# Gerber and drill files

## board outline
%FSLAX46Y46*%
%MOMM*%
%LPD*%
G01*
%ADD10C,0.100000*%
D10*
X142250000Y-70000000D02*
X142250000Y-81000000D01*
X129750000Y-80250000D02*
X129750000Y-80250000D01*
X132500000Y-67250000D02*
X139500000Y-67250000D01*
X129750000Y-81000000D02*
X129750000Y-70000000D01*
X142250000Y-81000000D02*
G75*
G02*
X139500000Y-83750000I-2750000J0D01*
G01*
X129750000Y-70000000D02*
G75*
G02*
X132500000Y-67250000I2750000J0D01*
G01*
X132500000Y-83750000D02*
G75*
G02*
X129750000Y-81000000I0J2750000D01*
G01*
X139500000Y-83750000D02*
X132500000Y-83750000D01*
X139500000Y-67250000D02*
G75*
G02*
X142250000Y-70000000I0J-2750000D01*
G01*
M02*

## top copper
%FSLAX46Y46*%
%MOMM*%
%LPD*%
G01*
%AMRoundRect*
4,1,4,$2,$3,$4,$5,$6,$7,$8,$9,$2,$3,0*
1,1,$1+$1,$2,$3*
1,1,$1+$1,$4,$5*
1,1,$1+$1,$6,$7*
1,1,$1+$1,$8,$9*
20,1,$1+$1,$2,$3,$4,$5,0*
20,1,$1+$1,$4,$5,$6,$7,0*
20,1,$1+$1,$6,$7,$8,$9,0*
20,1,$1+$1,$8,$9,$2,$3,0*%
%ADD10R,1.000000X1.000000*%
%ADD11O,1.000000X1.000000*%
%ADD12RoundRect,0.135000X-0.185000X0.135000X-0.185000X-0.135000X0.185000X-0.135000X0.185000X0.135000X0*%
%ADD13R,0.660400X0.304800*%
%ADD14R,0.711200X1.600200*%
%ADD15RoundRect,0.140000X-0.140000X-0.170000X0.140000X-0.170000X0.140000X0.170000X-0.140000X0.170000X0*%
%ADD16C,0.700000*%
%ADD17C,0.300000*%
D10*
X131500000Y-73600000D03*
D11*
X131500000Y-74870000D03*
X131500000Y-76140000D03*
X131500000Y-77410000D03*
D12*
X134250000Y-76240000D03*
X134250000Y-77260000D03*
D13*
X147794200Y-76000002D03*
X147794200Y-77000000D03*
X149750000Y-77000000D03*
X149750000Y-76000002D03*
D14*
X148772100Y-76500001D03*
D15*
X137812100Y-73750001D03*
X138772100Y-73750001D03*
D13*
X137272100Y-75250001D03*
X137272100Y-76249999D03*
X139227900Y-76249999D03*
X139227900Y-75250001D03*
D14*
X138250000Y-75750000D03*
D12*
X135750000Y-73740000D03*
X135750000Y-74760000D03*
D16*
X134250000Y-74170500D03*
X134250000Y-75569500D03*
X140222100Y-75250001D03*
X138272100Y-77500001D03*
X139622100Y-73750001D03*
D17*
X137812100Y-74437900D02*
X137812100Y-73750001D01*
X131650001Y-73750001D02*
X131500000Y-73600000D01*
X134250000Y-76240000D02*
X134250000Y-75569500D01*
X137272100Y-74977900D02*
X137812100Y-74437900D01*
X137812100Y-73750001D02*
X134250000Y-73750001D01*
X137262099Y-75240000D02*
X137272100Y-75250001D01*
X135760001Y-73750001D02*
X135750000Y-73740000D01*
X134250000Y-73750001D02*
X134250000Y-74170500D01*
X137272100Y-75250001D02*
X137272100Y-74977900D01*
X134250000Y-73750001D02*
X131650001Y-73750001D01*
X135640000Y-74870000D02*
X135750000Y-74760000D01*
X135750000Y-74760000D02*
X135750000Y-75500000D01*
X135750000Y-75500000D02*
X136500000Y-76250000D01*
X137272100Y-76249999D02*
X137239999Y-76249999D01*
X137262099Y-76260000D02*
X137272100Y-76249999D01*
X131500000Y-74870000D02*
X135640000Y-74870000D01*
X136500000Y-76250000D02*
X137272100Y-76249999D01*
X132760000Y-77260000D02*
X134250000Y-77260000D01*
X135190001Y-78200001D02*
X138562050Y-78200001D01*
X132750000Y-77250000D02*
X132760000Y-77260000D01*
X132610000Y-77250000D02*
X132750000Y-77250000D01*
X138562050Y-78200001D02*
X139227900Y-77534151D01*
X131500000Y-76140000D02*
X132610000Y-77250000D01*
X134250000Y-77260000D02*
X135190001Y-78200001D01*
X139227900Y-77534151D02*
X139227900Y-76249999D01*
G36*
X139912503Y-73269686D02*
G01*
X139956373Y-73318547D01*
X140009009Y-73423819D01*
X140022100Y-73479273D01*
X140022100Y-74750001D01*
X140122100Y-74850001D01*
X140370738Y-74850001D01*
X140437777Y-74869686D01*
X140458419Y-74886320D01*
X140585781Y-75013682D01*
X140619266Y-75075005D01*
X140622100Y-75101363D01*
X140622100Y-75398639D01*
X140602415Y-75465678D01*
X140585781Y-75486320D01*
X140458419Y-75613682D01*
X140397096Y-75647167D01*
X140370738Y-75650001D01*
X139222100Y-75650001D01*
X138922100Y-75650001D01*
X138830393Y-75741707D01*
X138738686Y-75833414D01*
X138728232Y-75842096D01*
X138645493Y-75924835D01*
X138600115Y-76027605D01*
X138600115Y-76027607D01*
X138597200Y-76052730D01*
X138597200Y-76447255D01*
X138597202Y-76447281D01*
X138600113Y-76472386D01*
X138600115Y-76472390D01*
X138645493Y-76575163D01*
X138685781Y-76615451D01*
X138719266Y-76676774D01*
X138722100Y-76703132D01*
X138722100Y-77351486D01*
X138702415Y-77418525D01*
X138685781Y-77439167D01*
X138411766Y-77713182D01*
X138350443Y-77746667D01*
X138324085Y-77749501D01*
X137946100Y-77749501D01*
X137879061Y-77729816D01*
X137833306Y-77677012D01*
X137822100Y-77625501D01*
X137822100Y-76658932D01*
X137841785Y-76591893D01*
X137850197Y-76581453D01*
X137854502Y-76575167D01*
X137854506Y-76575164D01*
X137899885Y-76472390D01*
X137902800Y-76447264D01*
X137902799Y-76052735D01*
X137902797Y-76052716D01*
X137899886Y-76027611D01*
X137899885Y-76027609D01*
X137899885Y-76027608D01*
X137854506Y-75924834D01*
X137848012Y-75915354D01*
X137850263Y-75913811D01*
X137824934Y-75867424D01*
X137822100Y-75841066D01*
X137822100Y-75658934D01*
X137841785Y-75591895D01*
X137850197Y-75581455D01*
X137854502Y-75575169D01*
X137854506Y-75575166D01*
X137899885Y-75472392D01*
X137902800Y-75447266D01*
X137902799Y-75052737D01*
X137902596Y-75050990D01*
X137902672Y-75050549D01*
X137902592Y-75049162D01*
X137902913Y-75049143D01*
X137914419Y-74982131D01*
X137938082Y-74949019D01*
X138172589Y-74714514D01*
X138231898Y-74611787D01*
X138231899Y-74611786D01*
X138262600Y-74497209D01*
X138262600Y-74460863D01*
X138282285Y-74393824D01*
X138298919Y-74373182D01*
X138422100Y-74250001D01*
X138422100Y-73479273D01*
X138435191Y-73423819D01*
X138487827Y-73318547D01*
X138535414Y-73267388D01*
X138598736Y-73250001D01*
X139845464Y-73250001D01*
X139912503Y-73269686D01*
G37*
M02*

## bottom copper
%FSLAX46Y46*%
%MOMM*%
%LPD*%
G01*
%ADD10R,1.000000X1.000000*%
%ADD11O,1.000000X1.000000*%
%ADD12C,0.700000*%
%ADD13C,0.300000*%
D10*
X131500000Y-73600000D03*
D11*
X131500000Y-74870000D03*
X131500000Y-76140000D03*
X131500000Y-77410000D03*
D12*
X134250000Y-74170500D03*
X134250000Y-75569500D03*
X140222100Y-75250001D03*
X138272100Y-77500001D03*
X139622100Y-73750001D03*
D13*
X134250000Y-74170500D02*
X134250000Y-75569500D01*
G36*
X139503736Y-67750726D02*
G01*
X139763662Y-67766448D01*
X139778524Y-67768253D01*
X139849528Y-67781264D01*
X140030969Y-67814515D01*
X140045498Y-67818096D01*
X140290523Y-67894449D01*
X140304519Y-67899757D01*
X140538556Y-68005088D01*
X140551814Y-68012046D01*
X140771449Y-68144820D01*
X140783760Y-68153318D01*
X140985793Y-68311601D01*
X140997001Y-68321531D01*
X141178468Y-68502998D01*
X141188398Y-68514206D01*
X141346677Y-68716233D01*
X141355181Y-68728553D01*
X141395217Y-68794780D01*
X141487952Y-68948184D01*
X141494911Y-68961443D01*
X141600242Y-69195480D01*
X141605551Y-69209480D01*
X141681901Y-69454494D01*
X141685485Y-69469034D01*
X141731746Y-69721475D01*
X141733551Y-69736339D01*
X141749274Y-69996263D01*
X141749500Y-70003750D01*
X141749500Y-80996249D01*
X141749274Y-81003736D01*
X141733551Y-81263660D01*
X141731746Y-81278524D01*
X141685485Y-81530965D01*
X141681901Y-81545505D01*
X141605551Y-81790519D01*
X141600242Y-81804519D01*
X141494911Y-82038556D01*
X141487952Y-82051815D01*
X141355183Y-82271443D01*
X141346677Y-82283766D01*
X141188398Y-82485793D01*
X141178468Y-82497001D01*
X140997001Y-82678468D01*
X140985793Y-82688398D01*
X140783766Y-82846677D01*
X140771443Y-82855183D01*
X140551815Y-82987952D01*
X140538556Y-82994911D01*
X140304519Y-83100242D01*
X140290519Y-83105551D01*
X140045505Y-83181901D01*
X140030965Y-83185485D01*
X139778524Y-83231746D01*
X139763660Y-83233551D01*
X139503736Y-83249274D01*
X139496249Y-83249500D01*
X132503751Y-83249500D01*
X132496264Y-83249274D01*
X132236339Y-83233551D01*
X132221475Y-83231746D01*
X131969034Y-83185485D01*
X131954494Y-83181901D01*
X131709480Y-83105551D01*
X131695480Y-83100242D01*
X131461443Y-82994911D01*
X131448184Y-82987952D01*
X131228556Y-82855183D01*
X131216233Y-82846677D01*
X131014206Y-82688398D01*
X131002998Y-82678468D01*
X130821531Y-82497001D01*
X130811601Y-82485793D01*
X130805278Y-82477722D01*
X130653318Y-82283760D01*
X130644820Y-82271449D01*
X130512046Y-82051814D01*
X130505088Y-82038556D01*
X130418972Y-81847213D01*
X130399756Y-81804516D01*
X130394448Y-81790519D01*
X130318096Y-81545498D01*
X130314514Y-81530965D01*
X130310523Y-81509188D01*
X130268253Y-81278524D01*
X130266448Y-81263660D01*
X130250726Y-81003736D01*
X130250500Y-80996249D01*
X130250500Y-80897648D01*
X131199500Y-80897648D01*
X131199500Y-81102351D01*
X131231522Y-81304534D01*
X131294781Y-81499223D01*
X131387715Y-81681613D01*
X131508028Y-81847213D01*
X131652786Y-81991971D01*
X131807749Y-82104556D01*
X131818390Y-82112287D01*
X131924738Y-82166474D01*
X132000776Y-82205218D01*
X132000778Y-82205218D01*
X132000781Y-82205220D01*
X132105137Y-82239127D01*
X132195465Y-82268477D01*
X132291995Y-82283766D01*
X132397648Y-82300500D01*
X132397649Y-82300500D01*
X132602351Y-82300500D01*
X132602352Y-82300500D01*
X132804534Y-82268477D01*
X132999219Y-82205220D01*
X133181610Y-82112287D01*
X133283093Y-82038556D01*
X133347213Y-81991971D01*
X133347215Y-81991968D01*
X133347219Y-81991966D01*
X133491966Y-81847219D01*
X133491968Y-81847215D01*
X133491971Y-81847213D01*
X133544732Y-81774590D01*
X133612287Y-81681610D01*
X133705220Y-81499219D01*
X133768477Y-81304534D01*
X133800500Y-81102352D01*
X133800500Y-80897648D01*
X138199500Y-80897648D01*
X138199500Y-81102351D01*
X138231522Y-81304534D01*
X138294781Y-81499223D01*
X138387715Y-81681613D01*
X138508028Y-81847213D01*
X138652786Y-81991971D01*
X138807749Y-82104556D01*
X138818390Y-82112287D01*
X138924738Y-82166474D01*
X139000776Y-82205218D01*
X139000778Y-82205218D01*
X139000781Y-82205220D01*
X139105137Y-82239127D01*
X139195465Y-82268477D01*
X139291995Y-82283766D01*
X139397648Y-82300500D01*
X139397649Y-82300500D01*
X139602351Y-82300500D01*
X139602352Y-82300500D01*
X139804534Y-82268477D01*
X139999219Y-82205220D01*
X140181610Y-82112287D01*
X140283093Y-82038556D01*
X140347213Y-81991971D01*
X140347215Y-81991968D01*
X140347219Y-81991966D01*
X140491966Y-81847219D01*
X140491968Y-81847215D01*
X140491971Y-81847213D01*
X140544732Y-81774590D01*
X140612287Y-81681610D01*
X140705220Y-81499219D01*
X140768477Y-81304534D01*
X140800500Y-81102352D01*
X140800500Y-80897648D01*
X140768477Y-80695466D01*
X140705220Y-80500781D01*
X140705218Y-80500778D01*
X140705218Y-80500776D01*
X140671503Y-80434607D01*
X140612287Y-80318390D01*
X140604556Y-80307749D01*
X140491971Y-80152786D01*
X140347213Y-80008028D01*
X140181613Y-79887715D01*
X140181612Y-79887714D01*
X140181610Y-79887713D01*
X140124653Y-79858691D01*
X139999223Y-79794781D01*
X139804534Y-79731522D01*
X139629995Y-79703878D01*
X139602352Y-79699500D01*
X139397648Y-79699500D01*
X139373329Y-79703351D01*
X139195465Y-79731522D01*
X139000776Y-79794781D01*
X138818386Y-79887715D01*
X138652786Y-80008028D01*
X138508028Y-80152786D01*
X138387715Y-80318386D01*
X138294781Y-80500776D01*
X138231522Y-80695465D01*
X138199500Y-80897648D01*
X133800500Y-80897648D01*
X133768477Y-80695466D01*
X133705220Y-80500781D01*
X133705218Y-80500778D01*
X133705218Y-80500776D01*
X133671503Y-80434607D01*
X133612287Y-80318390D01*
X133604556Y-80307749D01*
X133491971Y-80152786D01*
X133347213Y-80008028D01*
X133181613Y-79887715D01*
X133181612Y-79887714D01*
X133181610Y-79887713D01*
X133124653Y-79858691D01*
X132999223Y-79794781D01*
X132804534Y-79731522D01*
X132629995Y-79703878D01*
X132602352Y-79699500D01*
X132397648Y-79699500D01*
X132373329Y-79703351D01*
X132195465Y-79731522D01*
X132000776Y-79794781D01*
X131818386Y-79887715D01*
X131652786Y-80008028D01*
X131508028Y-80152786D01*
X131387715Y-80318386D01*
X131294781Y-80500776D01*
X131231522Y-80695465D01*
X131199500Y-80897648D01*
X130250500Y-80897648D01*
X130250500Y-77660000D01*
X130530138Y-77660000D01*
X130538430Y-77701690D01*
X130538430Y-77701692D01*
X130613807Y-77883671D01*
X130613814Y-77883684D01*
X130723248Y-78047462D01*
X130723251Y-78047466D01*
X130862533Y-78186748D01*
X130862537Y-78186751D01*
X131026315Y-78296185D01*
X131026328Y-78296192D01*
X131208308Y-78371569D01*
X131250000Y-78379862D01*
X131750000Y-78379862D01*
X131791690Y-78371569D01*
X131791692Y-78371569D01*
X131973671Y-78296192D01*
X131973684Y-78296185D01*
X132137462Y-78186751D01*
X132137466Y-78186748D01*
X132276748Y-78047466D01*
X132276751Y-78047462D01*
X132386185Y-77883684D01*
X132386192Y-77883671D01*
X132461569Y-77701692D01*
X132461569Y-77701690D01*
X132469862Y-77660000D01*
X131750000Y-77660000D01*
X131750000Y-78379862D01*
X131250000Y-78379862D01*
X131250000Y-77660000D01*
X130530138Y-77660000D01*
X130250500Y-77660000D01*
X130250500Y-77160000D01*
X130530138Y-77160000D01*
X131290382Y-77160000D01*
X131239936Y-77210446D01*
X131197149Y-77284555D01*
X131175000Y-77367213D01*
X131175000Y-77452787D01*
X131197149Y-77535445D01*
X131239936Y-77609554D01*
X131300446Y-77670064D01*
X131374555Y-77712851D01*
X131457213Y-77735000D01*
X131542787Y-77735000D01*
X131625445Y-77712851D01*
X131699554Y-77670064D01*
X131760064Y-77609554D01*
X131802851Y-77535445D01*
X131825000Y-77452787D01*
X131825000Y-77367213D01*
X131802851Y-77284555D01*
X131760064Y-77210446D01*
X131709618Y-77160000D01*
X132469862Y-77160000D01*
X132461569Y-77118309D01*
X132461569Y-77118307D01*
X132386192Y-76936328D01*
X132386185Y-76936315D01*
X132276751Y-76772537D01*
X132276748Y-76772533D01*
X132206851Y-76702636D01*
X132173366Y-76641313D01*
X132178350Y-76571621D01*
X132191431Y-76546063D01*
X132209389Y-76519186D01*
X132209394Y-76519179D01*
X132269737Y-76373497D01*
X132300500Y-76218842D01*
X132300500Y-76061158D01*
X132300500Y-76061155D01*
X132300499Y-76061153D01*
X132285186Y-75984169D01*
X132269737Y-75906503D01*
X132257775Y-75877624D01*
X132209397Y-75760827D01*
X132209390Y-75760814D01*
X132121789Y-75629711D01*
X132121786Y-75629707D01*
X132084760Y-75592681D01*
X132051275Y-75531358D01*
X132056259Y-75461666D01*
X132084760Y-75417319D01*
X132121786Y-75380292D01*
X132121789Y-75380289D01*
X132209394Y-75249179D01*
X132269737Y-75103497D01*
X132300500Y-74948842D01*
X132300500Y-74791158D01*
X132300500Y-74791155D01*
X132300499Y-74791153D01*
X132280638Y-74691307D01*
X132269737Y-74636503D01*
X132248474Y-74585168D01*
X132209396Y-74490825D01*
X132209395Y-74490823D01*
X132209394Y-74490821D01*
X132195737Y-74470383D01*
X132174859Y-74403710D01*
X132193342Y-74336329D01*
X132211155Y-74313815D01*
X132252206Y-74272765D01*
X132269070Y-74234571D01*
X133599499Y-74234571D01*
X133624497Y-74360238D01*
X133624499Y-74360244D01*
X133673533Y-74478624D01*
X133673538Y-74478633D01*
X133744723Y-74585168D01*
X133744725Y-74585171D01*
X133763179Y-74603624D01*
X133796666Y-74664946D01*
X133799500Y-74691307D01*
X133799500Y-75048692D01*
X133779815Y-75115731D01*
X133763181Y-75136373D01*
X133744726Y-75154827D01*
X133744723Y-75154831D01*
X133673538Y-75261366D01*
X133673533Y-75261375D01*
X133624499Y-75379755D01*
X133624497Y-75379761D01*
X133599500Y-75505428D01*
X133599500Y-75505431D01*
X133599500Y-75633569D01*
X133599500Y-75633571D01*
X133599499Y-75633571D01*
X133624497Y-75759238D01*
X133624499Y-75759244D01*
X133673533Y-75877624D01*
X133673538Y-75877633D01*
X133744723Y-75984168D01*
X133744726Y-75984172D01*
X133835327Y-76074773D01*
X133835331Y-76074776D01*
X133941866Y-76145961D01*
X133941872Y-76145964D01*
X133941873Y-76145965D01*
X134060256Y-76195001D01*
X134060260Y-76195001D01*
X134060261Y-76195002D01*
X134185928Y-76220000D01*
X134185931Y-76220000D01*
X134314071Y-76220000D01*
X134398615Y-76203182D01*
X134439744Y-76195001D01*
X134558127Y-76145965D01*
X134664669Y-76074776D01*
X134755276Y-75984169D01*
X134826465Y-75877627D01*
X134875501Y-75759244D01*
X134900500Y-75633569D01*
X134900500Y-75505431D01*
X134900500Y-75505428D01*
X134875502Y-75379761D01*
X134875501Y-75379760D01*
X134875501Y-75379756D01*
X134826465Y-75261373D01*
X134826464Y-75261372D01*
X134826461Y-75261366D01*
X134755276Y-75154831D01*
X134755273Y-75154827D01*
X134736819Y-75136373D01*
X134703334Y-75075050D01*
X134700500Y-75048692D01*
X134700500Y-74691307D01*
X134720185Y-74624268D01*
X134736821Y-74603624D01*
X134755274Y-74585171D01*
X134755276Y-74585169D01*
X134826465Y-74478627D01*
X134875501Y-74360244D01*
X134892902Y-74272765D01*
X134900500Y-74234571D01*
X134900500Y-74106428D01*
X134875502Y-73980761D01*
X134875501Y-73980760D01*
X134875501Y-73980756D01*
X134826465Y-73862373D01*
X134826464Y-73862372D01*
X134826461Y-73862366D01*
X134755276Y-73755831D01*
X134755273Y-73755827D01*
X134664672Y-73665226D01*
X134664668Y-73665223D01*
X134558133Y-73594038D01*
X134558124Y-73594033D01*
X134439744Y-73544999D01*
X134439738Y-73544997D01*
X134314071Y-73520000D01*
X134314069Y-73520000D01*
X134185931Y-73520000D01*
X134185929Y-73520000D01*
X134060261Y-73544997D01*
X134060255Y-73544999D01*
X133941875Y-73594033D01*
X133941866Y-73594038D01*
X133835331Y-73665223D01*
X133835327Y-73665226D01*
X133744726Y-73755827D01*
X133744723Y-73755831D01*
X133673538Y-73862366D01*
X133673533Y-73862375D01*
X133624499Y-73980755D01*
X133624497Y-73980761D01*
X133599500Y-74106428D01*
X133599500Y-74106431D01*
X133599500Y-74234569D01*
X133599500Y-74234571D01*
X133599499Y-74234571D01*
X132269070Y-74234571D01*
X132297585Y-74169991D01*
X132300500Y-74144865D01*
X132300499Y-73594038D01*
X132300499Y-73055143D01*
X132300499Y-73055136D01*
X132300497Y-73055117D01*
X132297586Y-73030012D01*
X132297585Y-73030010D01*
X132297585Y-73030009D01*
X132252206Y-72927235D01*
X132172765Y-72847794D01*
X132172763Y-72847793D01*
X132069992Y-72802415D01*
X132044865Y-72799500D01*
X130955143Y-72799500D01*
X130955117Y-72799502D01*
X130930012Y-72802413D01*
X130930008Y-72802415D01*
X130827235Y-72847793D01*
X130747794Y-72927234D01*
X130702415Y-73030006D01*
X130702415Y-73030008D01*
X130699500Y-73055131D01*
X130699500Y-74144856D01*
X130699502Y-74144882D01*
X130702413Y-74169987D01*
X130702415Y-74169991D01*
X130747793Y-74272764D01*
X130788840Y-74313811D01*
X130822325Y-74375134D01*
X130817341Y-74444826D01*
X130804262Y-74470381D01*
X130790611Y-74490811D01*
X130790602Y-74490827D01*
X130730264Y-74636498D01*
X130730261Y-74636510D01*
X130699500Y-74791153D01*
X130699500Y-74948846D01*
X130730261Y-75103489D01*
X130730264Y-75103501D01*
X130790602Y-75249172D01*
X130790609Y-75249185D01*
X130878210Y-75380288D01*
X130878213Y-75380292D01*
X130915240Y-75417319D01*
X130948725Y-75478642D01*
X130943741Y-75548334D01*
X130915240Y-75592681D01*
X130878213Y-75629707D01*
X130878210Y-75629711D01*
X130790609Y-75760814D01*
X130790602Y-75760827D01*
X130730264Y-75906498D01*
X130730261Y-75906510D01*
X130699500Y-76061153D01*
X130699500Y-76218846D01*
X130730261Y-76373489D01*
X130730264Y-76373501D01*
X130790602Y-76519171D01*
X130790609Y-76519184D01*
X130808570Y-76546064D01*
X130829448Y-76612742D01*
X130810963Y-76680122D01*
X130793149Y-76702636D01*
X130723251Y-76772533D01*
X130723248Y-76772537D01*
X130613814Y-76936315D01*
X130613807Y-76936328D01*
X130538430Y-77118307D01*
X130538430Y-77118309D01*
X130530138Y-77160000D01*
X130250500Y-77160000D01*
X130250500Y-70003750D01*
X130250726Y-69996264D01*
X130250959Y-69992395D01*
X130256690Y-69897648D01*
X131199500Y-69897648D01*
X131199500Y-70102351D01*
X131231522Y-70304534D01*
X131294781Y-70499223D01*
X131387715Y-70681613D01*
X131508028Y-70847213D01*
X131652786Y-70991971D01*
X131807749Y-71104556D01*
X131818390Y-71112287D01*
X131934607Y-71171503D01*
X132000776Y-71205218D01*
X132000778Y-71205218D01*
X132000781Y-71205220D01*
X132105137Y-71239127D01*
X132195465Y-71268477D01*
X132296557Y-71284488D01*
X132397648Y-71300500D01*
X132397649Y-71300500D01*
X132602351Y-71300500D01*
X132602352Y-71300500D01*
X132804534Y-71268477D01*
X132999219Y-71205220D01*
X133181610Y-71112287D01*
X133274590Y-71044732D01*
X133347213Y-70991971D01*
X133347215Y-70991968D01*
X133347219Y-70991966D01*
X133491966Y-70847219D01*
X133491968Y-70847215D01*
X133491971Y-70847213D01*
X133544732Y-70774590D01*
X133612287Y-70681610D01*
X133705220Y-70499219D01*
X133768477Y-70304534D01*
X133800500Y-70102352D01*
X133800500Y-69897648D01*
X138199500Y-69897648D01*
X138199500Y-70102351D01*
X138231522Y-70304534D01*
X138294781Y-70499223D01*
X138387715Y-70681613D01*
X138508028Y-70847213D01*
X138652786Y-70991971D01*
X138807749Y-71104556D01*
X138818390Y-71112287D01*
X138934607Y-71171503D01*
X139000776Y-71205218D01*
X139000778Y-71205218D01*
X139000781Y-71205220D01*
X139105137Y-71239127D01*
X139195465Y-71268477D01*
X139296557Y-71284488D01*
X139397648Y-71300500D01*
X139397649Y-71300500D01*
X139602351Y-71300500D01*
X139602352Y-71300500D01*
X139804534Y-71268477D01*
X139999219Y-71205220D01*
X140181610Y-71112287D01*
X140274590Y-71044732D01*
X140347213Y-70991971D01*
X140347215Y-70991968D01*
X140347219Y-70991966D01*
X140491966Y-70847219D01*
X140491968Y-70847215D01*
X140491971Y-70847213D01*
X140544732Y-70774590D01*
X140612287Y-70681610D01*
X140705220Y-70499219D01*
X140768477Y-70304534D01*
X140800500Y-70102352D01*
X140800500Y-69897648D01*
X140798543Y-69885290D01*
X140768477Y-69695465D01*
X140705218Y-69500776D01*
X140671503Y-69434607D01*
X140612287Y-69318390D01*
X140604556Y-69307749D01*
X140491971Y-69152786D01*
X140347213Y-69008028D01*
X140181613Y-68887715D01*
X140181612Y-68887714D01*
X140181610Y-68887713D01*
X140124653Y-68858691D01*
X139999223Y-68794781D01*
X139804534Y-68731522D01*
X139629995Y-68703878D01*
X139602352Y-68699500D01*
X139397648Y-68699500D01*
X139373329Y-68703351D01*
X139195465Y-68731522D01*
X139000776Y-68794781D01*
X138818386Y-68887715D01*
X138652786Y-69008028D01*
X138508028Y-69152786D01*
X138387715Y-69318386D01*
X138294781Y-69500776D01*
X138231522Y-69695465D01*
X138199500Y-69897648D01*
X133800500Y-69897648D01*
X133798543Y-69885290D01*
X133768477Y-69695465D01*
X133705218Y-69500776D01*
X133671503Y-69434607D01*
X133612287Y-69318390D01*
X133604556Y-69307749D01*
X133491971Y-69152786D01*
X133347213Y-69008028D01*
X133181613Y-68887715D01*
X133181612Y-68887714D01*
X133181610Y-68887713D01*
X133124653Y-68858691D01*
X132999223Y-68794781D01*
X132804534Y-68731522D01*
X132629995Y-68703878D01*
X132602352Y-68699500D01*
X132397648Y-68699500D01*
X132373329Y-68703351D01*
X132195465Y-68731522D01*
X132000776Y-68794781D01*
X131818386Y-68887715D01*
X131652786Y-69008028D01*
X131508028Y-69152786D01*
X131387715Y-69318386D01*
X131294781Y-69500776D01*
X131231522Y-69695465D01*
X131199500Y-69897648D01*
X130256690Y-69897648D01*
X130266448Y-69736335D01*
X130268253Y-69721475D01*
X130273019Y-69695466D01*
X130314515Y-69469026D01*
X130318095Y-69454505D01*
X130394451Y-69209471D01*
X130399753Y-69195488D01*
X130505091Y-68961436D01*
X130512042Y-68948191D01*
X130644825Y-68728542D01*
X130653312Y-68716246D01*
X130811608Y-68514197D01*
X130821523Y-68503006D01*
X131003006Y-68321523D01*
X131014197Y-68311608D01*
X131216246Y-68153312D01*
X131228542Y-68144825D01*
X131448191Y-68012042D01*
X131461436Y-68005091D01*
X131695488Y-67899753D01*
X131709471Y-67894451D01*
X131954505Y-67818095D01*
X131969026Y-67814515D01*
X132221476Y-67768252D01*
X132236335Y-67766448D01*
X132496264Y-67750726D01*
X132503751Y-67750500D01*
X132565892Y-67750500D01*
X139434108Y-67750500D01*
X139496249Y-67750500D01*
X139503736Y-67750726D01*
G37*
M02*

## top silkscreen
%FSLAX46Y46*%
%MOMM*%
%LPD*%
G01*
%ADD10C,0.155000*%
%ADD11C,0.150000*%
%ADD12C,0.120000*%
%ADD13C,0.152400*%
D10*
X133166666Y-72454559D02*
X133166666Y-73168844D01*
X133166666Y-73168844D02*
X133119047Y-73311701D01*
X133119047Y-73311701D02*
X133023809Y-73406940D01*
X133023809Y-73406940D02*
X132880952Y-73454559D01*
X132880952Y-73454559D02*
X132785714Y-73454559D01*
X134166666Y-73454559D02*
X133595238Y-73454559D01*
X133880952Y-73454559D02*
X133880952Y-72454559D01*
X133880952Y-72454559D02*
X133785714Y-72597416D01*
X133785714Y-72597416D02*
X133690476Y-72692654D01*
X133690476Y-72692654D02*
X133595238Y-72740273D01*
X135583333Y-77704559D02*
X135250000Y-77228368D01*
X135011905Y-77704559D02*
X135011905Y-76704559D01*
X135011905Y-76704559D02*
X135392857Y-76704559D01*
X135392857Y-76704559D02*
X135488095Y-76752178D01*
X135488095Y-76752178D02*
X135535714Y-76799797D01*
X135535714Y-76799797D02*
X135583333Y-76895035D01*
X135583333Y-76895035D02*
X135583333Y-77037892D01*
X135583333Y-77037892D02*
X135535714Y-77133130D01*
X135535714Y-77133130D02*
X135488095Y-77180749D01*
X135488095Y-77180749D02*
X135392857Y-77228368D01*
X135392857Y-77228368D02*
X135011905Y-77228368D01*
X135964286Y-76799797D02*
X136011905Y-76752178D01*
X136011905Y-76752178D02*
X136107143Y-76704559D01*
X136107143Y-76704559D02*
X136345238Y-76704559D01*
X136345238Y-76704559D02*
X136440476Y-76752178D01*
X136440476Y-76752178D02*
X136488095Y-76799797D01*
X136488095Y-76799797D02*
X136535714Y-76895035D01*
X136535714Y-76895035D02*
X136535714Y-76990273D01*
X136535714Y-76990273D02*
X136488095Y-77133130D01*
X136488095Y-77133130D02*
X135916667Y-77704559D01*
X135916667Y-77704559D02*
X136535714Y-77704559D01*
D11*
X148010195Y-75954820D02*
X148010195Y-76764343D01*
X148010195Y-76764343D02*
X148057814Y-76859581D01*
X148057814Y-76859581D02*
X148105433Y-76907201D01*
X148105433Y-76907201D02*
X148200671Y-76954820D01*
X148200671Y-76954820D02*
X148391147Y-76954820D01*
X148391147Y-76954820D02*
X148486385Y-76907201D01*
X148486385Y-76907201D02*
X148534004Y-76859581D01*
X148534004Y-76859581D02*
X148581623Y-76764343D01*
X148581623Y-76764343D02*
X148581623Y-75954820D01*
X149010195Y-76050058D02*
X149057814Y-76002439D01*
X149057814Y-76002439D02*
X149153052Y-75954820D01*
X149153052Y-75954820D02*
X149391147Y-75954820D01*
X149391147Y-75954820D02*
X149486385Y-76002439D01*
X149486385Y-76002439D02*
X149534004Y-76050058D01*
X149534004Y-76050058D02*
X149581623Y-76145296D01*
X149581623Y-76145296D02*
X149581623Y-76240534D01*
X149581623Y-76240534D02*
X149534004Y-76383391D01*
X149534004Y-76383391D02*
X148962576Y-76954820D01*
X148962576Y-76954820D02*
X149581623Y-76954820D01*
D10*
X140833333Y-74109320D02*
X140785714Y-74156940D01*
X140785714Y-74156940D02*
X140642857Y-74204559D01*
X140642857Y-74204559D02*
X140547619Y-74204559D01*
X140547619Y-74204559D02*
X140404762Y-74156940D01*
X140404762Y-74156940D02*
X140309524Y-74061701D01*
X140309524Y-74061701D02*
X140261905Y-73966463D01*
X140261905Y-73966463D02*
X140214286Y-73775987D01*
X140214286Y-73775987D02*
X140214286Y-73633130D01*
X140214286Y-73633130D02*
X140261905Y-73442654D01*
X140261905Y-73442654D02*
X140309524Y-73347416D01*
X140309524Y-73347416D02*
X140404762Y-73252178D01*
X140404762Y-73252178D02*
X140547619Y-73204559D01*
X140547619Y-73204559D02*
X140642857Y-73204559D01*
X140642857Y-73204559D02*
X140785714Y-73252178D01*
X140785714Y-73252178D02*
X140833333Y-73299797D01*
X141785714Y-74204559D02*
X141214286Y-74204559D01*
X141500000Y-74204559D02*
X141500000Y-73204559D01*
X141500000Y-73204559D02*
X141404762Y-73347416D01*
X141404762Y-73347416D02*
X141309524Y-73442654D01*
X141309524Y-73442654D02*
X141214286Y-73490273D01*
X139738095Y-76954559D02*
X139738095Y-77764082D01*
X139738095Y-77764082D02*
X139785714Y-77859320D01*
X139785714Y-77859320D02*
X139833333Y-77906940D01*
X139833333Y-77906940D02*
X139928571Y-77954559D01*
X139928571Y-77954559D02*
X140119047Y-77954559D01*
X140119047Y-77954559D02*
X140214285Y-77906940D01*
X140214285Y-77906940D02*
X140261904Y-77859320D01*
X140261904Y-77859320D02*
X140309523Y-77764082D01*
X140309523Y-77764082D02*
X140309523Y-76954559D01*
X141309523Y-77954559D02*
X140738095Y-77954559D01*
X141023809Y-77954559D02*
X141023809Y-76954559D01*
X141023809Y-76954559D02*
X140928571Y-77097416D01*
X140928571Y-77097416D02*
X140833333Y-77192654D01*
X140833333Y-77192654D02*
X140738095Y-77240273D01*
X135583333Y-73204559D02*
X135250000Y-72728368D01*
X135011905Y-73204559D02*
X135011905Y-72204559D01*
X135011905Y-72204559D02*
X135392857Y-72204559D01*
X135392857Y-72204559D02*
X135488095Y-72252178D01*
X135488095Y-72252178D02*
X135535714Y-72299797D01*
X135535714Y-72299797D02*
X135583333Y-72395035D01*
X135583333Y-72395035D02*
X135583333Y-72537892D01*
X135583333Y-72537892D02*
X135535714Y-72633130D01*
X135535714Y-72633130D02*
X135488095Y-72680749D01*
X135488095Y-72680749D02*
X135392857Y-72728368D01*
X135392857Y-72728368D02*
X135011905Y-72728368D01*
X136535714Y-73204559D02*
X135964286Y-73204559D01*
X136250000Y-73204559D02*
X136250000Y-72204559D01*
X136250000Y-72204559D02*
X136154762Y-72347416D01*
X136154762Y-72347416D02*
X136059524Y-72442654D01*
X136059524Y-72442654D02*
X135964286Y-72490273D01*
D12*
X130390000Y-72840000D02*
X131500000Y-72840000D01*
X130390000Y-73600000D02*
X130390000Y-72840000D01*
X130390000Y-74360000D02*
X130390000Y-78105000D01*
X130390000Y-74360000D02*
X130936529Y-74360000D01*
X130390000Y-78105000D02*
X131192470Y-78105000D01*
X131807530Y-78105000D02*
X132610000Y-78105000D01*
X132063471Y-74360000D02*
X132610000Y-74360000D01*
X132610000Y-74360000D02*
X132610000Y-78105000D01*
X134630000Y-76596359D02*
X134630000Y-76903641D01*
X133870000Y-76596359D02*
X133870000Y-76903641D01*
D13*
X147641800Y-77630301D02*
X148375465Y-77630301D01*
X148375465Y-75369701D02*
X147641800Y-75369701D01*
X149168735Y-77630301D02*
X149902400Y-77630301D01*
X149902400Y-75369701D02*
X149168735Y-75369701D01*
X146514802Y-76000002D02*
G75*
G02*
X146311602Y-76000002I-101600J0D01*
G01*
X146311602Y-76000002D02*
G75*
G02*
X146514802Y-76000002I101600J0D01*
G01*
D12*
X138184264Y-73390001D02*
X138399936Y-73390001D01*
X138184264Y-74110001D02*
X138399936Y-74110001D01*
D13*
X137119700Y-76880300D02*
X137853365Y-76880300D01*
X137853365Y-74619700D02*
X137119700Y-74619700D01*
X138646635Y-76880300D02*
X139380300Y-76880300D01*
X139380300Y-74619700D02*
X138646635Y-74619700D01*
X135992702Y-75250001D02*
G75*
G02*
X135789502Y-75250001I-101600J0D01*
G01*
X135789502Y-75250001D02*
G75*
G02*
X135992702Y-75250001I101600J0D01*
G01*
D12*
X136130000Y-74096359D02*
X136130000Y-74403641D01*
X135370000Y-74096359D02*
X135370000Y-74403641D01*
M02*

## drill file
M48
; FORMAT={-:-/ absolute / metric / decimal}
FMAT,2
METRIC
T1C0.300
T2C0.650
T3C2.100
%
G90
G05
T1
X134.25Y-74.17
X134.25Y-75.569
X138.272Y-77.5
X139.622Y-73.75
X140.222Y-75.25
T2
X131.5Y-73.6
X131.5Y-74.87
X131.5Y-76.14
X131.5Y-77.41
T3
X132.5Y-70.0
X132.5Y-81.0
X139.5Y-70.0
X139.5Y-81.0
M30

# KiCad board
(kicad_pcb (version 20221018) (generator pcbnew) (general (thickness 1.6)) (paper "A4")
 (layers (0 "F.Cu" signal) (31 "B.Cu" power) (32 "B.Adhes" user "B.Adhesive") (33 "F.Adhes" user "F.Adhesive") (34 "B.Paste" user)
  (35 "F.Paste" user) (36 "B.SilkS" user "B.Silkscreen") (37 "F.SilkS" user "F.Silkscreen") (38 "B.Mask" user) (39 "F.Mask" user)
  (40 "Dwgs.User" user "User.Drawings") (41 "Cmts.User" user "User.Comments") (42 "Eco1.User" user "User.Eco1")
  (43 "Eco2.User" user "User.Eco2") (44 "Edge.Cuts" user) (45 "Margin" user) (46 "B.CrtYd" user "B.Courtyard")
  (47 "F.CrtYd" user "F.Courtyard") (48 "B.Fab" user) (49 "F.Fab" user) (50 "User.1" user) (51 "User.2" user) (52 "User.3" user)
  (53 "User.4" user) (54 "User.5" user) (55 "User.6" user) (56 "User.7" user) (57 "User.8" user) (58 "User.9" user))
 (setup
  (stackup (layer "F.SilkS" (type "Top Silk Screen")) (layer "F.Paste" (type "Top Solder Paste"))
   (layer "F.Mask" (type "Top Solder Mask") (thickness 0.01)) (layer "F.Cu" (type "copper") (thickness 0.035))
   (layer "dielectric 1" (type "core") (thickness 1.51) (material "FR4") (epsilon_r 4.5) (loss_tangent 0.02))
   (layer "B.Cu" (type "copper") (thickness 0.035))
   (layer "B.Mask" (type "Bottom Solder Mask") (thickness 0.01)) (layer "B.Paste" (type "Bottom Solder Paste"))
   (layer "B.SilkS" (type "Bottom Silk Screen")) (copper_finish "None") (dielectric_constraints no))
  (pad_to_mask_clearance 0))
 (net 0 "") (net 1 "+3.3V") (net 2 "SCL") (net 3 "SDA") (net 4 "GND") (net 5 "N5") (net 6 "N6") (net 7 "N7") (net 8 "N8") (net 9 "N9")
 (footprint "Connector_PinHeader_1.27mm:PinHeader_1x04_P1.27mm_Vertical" (layer "F.Cu") (at 131.5 73.6)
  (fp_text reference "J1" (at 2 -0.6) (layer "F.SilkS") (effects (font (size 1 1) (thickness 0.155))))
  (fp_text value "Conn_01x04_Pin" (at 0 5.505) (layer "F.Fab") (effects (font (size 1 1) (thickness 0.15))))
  (fp_line (start -1.11 -0.76) (end 0 -0.76) (stroke (width 0.12) (type solid)) (layer "F.SilkS"))
  (fp_line (start -1.11 0) (end -1.11 -0.76) (stroke (width 0.12) (type solid)) (layer "F.SilkS"))
  (fp_line (start -1.11 0.76) (end -1.11 4.505) (stroke (width 0.12) (type solid)) (layer "F.SilkS"))
  (fp_line (start -1.11 0.76) (end -0.563471 0.76) (stroke (width 0.12) (type solid)) (layer "F.SilkS"))
  (fp_line (start -1.11 4.505) (end -0.30753 4.505) (stroke (width 0.12) (type solid)) (layer "F.SilkS"))
  (fp_line (start 0.30753 4.505) (end 1.11 4.505) (stroke (width 0.12) (type solid)) (layer "F.SilkS"))
  (fp_line (start 0.563471 0.76) (end 1.11 0.76) (stroke (width 0.12) (type solid)) (layer "F.SilkS"))
  (fp_line (start 1.11 0.76) (end 1.11 4.505) (stroke (width 0.12) (type solid)) (layer "F.SilkS"))
  (pad "1" thru_hole rect (at 0 0) (size 1 1) (drill 0.65) (layers "*.Cu" "*.Mask") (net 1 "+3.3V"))
  (pad "2" thru_hole oval (at 0 1.27) (size 1 1) (drill 0.65) (layers "*.Cu" "*.Mask") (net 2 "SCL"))
  (pad "3" thru_hole oval (at 0 2.54) (size 1 1) (drill 0.65) (layers "*.Cu" "*.Mask") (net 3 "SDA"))
  (pad "4" thru_hole oval (at 0 3.81) (size 1 1) (drill 0.65) (layers "*.Cu" "*.Mask") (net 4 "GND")))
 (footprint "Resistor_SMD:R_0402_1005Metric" (layer "F.Cu") (at 134.25 76.75 -90)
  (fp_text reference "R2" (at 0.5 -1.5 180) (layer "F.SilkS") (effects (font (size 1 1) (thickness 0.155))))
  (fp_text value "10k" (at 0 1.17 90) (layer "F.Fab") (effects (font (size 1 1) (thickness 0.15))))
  (fp_line (start -0.153641 -0.38) (end 0.153641 -0.38) (stroke (width 0.12) (type solid)) (layer "F.SilkS"))
  (fp_line (start -0.153641 0.38) (end 0.153641 0.38) (stroke (width 0.12) (type solid)) (layer "F.SilkS"))
  (pad "1" smd roundrect (at -0.51 0 270) (size 0.54 0.64) (layers "F.Cu" "F.Paste" "F.Mask") (roundrect_rratio 0.25) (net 1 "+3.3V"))
  (pad "2" smd roundrect (at 0.51 0 270) (size 0.54 0.64) (layers "F.Cu" "F.Paste" "F.Mask") (roundrect_rratio 0.25) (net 3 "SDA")))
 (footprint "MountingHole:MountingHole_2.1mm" (layer "F.Cu") (at 139.5 70)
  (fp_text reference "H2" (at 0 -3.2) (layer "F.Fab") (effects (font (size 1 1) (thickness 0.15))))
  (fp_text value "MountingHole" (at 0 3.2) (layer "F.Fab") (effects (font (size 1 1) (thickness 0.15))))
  (pad "" np_thru_hole circle (at 0 0) (size 2.1 2.1) (drill 2.1) (layers "*.Cu" "*.Mask")))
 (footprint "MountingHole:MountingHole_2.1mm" (layer "F.Cu") (at 132.5 81)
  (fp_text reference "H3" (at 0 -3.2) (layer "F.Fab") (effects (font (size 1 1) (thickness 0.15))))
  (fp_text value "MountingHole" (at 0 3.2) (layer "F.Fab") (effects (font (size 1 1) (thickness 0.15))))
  (pad "" np_thru_hole circle (at 0 0) (size 2.1 2.1) (drill 2.1) (layers "*.Cu" "*.Mask")))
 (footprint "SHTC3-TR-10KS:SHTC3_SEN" (layer "F.Cu") (at 148.7721 76.500001)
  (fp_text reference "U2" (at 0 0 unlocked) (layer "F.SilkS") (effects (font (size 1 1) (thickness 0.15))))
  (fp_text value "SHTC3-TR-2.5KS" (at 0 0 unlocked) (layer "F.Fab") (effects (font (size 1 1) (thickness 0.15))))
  (fp_line (start -1.1303 1.1303) (end -0.396635 1.1303) (stroke (width 0.1524) (type solid)) (layer "F.SilkS"))
  (fp_line (start -0.396635 -1.1303) (end -1.1303 -1.1303) (stroke (width 0.1524) (type solid)) (layer "F.SilkS"))
  (fp_line (start 0.396635 1.1303) (end 1.1303 1.1303) (stroke (width 0.1524) (type solid)) (layer "F.SilkS"))
  (fp_line (start 1.1303 -1.1303) (end 0.396635 -1.1303) (stroke (width 0.1524) (type solid)) (layer "F.SilkS"))
  (fp_circle (center -2.358898 -0.499999) (end -2.257298 -0.499999) (stroke (width 0.1524) (type solid)) (fill none) (layer "F.SilkS"))
  (pad "1" smd rect (at -0.9779 -0.499999) (size 0.6604 0.3048) (layers "F.Cu" "F.Paste" "F.Mask") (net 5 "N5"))
  (pad "2" smd rect (at -0.9779 0.499999) (size 0.6604 0.3048) (layers "F.Cu" "F.Paste" "F.Mask") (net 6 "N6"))
  (pad "3" smd rect (at 0.9779 0.499999) (size 0.6604 0.3048) (layers "F.Cu" "F.Paste" "F.Mask") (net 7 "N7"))
  (pad "4" smd rect (at 0.9779 -0.499999) (size 0.6604 0.3048) (layers "F.Cu" "F.Paste" "F.Mask") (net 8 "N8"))
  (pad "5" smd rect (at 0 0) (size 0.7112 1.6002) (layers "F.Cu" "F.Paste" "F.Mask") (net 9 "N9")))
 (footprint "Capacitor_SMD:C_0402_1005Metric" (layer "F.Cu") (at 138.2921 73.750001)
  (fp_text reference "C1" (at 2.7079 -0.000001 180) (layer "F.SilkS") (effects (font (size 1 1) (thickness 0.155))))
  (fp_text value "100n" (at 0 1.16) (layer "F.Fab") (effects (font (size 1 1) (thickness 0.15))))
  (fp_line (start -0.107836 -0.36) (end 0.107836 -0.36) (stroke (width 0.12) (type solid)) (layer "F.SilkS"))
  (fp_line (start -0.107836 0.36) (end 0.107836 0.36) (stroke (width 0.12) (type solid)) (layer "F.SilkS"))
  (pad "1" smd roundrect (at -0.48 0) (size 0.56 0.62) (layers "F.Cu" "F.Paste" "F.Mask") (roundrect_rratio 0.25) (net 1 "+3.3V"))
  (pad "2" smd roundrect (at 0.48 0) (size 0.56 0.62) (layers "F.Cu" "F.Paste" "F.Mask") (roundrect_rratio 0.25) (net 4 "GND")))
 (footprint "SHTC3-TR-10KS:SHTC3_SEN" (layer "F.Cu") (at 138.25 75.75)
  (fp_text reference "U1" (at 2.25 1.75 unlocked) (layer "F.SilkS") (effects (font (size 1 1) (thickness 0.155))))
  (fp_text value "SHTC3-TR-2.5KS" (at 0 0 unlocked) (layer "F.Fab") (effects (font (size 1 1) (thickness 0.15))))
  (fp_line (start -1.1303 1.1303) (end -0.396635 1.1303) (stroke (width 0.1524) (type solid)) (layer "F.SilkS"))
  (fp_line (start -0.396635 -1.1303) (end -1.1303 -1.1303) (stroke (width 0.1524) (type solid)) (layer "F.SilkS"))
  (fp_line (start 0.396635 1.1303) (end 1.1303 1.1303) (stroke (width 0.1524) (type solid)) (layer "F.SilkS"))
  (fp_line (start 1.1303 -1.1303) (end 0.396635 -1.1303) (stroke (width 0.1524) (type solid)) (layer "F.SilkS"))
  (fp_circle (center -2.358898 -0.499999) (end -2.257298 -0.499999) (stroke (width 0.1524) (type solid)) (fill none) (layer "F.SilkS"))
  (pad "1" smd rect (at -0.9779 -0.499999) (size 0.6604 0.3048) (layers "F.Cu" "F.Paste" "F.Mask") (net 1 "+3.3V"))
  (pad "2" smd rect (at -0.9779 0.499999) (size 0.6604 0.3048) (layers "F.Cu" "F.Paste" "F.Mask") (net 2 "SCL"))
  (pad "3" smd rect (at 0.9779 0.499999) (size 0.6604 0.3048) (layers "F.Cu" "F.Paste" "F.Mask") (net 3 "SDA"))
  (pad "4" smd rect (at 0.9779 -0.499999) (size 0.6604 0.3048) (layers "F.Cu" "F.Paste" "F.Mask") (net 4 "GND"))
  (pad "5" smd rect (at 0 0) (size 0.7112 1.6002) (layers "F.Cu" "F.Paste" "F.Mask") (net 4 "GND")))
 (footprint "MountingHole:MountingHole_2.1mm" (layer "F.Cu") (at 139.5 81)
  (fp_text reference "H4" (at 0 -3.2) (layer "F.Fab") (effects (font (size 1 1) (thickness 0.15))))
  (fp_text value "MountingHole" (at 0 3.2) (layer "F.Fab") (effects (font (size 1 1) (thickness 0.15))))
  (pad "" np_thru_hole circle (at 0 0) (size 2.1 2.1) (drill 2.1) (layers "*.Cu" "*.Mask")))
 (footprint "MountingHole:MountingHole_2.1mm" (layer "F.Cu") (at 132.5 70)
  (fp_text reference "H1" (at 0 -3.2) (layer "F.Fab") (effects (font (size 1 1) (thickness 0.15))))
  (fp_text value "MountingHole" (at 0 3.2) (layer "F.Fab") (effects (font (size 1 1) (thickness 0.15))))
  (pad "" np_thru_hole circle (at 0 0) (size 2.1 2.1) (drill 2.1) (layers "*.Cu" "*.Mask")))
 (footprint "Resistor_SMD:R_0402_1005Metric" (layer "F.Cu") (at 135.75 74.25 -90)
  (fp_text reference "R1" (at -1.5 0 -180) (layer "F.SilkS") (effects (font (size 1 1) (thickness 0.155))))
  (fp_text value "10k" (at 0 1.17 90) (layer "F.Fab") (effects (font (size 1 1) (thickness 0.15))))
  (fp_line (start -0.153641 -0.38) (end 0.153641 -0.38) (stroke (width 0.12) (type solid)) (layer "F.SilkS"))
  (fp_line (start -0.153641 0.38) (end 0.153641 0.38) (stroke (width 0.12) (type solid)) (layer "F.SilkS"))
  (pad "1" smd roundrect (at -0.51 0 270) (size 0.54 0.64) (layers "F.Cu" "F.Paste" "F.Mask") (roundrect_rratio 0.25) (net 1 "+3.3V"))
  (pad "2" smd roundrect (at 0.51 0 270) (size 0.54 0.64) (layers "F.Cu" "F.Paste" "F.Mask") (roundrect_rratio 0.25) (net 2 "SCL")))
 (gr_line (start 142.25 70) (end 142.25 81) (stroke (width 0.1) (type default)) (layer "Edge.Cuts"))
 (gr_line (start 129.75 80.25) (end 129.75 80.25) (stroke (width 0.1) (type default)) (layer "Edge.Cuts"))
 (gr_line (start 132.5 67.25) (end 139.5 67.25) (stroke (width 0.1) (type default)) (layer "Edge.Cuts"))
 (gr_line (start 129.75 81) (end 129.75 70) (stroke (width 0.1) (type default)) (layer "Edge.Cuts"))
 (gr_arc (start 142.25 81) (mid 141.444544 82.944544) (end 139.5 83.75) (stroke (width 0.1) (type default)) (layer "Edge.Cuts"))
 (gr_arc (start 129.75 70) (mid 130.555456 68.055456) (end 132.5 67.25) (stroke (width 0.1) (type default)) (layer "Edge.Cuts"))
 (gr_arc (start 132.5 83.75) (mid 130.555456 82.944544) (end 129.75 81) (stroke (width 0.1) (type default)) (layer "Edge.Cuts"))
 (gr_line (start 139.5 83.75) (end 132.5 83.75) (stroke (width 0.1) (type default)) (layer "Edge.Cuts"))
 (gr_arc (start 139.5 67.25) (mid 141.444544 68.055456) (end 142.25 70) (stroke (width 0.1) (type default)) (layer "Edge.Cuts"))
 (segment (start 137.8121 74.4379) (end 137.8121 73.750001) (width 0.3) (layer "F.Cu") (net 1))
 (segment (start 131.650001 73.750001) (end 131.5 73.6) (width 0.3) (layer "F.Cu") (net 1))
 (segment (start 134.25 76.24) (end 134.25 75.5695) (width 0.3) (layer "F.Cu") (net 1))
 (segment (start 137.2721 74.9779) (end 137.8121 74.4379) (width 0.3) (layer "F.Cu") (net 1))
 (segment (start 137.8121 73.750001) (end 134.25 73.750001) (width 0.3) (layer "F.Cu") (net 1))
 (segment (start 137.262099 75.24) (end 137.2721 75.250001) (width 0.3) (layer "F.Cu") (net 1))
 (segment (start 135.760001 73.750001) (end 135.75 73.74) (width 0.3) (layer "F.Cu") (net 1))
 (segment (start 134.25 73.750001) (end 134.25 74.1705) (width 0.3) (layer "F.Cu") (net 1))
 (segment (start 137.2721 75.250001) (end 137.2721 74.9779) (width 0.3) (layer "F.Cu") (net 1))
 (segment (start 134.25 73.750001) (end 131.650001 73.750001) (width 0.3) (layer "F.Cu") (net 1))
 (via (at 134.25 74.1705) (size 0.7) (drill 0.3) (layers "F.Cu" "B.Cu") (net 1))
 (via (at 134.25 75.5695) (size 0.7) (drill 0.3) (layers "F.Cu" "B.Cu") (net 1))
 (segment (start 134.25 74.1705) (end 134.25 75.5695) (width 0.3) (layer "B.Cu") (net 1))
 (via (at 140.2221 75.250001) (size 0.7) (drill 0.3) (layers "F.Cu" "B.Cu") (free) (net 4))
 (via (at 138.2721 77.500001) (size 0.7) (drill 0.3) (layers "F.Cu" "B.Cu") (free) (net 4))
 (via (at 139.6221 73.750001) (size 0.7) (drill 0.3) (layers "F.Cu" "B.Cu") (free) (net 4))
 (segment (start 135.64 74.87) (end 135.75 74.76) (width 0.3) (layer "F.Cu") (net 2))
 (segment (start 135.75 74.76) (end 135.75 75.5) (width 0.3) (layer "F.Cu") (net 2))
 (segment (start 135.75 75.5) (end 136.5 76.25) (width 0.3) (layer "F.Cu") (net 2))
 (segment (start 137.2721 76.249999) (end 137.239999 76.249999) (width 0.3) (layer "F.Cu") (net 2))
 (segment (start 137.262099 76.26) (end 137.2721 76.249999) (width 0.3) (layer "F.Cu") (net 2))
 (segment (start 131.5 74.87) (end 135.64 74.87) (width 0.3) (layer "F.Cu") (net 2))
 (segment (start 136.5 76.25) (end 137.2721 76.249999) (width 0.3) (layer "F.Cu") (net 2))
 (segment (start 132.76 77.26) (end 134.25 77.26) (width 0.3) (layer "F.Cu") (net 3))
 (segment (start 135.190001 78.200001) (end 138.56205 78.200001) (width 0.3) (layer "F.Cu") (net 3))
 (segment (start 132.75 77.25) (end 132.76 77.26) (width 0.3) (layer "F.Cu") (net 3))
 (segment (start 132.61 77.25) (end 132.75 77.25) (width 0.3) (layer "F.Cu") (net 3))
 (segment (start 138.56205 78.200001) (end 139.2279 77.534151) (width 0.3) (layer "F.Cu") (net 3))
 (segment (start 131.5 76.14) (end 132.61 77.25) (width 0.3) (layer "F.Cu") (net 3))
 (segment (start 134.25 77.26) (end 135.190001 78.200001) (width 0.3) (layer "F.Cu") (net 3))
 (segment (start 139.2279 77.534151) (end 139.2279 76.249999) (width 0.3) (layer "F.Cu") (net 3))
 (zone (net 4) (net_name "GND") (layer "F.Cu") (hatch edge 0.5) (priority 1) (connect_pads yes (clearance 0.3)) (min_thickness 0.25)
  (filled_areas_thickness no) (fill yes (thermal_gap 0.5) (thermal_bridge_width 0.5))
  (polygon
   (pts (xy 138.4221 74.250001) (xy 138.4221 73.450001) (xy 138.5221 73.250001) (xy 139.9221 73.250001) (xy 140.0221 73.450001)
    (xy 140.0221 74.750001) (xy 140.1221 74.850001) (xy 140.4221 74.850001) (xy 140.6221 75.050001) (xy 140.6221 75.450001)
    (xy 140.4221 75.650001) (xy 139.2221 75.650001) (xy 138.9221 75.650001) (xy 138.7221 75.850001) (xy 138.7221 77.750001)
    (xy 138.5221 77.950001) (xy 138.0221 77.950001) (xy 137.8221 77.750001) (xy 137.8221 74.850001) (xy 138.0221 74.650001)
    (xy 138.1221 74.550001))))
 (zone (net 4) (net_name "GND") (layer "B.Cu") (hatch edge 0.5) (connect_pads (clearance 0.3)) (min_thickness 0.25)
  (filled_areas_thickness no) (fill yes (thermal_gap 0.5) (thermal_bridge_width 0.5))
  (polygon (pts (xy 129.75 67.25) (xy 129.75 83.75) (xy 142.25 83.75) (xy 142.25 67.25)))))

